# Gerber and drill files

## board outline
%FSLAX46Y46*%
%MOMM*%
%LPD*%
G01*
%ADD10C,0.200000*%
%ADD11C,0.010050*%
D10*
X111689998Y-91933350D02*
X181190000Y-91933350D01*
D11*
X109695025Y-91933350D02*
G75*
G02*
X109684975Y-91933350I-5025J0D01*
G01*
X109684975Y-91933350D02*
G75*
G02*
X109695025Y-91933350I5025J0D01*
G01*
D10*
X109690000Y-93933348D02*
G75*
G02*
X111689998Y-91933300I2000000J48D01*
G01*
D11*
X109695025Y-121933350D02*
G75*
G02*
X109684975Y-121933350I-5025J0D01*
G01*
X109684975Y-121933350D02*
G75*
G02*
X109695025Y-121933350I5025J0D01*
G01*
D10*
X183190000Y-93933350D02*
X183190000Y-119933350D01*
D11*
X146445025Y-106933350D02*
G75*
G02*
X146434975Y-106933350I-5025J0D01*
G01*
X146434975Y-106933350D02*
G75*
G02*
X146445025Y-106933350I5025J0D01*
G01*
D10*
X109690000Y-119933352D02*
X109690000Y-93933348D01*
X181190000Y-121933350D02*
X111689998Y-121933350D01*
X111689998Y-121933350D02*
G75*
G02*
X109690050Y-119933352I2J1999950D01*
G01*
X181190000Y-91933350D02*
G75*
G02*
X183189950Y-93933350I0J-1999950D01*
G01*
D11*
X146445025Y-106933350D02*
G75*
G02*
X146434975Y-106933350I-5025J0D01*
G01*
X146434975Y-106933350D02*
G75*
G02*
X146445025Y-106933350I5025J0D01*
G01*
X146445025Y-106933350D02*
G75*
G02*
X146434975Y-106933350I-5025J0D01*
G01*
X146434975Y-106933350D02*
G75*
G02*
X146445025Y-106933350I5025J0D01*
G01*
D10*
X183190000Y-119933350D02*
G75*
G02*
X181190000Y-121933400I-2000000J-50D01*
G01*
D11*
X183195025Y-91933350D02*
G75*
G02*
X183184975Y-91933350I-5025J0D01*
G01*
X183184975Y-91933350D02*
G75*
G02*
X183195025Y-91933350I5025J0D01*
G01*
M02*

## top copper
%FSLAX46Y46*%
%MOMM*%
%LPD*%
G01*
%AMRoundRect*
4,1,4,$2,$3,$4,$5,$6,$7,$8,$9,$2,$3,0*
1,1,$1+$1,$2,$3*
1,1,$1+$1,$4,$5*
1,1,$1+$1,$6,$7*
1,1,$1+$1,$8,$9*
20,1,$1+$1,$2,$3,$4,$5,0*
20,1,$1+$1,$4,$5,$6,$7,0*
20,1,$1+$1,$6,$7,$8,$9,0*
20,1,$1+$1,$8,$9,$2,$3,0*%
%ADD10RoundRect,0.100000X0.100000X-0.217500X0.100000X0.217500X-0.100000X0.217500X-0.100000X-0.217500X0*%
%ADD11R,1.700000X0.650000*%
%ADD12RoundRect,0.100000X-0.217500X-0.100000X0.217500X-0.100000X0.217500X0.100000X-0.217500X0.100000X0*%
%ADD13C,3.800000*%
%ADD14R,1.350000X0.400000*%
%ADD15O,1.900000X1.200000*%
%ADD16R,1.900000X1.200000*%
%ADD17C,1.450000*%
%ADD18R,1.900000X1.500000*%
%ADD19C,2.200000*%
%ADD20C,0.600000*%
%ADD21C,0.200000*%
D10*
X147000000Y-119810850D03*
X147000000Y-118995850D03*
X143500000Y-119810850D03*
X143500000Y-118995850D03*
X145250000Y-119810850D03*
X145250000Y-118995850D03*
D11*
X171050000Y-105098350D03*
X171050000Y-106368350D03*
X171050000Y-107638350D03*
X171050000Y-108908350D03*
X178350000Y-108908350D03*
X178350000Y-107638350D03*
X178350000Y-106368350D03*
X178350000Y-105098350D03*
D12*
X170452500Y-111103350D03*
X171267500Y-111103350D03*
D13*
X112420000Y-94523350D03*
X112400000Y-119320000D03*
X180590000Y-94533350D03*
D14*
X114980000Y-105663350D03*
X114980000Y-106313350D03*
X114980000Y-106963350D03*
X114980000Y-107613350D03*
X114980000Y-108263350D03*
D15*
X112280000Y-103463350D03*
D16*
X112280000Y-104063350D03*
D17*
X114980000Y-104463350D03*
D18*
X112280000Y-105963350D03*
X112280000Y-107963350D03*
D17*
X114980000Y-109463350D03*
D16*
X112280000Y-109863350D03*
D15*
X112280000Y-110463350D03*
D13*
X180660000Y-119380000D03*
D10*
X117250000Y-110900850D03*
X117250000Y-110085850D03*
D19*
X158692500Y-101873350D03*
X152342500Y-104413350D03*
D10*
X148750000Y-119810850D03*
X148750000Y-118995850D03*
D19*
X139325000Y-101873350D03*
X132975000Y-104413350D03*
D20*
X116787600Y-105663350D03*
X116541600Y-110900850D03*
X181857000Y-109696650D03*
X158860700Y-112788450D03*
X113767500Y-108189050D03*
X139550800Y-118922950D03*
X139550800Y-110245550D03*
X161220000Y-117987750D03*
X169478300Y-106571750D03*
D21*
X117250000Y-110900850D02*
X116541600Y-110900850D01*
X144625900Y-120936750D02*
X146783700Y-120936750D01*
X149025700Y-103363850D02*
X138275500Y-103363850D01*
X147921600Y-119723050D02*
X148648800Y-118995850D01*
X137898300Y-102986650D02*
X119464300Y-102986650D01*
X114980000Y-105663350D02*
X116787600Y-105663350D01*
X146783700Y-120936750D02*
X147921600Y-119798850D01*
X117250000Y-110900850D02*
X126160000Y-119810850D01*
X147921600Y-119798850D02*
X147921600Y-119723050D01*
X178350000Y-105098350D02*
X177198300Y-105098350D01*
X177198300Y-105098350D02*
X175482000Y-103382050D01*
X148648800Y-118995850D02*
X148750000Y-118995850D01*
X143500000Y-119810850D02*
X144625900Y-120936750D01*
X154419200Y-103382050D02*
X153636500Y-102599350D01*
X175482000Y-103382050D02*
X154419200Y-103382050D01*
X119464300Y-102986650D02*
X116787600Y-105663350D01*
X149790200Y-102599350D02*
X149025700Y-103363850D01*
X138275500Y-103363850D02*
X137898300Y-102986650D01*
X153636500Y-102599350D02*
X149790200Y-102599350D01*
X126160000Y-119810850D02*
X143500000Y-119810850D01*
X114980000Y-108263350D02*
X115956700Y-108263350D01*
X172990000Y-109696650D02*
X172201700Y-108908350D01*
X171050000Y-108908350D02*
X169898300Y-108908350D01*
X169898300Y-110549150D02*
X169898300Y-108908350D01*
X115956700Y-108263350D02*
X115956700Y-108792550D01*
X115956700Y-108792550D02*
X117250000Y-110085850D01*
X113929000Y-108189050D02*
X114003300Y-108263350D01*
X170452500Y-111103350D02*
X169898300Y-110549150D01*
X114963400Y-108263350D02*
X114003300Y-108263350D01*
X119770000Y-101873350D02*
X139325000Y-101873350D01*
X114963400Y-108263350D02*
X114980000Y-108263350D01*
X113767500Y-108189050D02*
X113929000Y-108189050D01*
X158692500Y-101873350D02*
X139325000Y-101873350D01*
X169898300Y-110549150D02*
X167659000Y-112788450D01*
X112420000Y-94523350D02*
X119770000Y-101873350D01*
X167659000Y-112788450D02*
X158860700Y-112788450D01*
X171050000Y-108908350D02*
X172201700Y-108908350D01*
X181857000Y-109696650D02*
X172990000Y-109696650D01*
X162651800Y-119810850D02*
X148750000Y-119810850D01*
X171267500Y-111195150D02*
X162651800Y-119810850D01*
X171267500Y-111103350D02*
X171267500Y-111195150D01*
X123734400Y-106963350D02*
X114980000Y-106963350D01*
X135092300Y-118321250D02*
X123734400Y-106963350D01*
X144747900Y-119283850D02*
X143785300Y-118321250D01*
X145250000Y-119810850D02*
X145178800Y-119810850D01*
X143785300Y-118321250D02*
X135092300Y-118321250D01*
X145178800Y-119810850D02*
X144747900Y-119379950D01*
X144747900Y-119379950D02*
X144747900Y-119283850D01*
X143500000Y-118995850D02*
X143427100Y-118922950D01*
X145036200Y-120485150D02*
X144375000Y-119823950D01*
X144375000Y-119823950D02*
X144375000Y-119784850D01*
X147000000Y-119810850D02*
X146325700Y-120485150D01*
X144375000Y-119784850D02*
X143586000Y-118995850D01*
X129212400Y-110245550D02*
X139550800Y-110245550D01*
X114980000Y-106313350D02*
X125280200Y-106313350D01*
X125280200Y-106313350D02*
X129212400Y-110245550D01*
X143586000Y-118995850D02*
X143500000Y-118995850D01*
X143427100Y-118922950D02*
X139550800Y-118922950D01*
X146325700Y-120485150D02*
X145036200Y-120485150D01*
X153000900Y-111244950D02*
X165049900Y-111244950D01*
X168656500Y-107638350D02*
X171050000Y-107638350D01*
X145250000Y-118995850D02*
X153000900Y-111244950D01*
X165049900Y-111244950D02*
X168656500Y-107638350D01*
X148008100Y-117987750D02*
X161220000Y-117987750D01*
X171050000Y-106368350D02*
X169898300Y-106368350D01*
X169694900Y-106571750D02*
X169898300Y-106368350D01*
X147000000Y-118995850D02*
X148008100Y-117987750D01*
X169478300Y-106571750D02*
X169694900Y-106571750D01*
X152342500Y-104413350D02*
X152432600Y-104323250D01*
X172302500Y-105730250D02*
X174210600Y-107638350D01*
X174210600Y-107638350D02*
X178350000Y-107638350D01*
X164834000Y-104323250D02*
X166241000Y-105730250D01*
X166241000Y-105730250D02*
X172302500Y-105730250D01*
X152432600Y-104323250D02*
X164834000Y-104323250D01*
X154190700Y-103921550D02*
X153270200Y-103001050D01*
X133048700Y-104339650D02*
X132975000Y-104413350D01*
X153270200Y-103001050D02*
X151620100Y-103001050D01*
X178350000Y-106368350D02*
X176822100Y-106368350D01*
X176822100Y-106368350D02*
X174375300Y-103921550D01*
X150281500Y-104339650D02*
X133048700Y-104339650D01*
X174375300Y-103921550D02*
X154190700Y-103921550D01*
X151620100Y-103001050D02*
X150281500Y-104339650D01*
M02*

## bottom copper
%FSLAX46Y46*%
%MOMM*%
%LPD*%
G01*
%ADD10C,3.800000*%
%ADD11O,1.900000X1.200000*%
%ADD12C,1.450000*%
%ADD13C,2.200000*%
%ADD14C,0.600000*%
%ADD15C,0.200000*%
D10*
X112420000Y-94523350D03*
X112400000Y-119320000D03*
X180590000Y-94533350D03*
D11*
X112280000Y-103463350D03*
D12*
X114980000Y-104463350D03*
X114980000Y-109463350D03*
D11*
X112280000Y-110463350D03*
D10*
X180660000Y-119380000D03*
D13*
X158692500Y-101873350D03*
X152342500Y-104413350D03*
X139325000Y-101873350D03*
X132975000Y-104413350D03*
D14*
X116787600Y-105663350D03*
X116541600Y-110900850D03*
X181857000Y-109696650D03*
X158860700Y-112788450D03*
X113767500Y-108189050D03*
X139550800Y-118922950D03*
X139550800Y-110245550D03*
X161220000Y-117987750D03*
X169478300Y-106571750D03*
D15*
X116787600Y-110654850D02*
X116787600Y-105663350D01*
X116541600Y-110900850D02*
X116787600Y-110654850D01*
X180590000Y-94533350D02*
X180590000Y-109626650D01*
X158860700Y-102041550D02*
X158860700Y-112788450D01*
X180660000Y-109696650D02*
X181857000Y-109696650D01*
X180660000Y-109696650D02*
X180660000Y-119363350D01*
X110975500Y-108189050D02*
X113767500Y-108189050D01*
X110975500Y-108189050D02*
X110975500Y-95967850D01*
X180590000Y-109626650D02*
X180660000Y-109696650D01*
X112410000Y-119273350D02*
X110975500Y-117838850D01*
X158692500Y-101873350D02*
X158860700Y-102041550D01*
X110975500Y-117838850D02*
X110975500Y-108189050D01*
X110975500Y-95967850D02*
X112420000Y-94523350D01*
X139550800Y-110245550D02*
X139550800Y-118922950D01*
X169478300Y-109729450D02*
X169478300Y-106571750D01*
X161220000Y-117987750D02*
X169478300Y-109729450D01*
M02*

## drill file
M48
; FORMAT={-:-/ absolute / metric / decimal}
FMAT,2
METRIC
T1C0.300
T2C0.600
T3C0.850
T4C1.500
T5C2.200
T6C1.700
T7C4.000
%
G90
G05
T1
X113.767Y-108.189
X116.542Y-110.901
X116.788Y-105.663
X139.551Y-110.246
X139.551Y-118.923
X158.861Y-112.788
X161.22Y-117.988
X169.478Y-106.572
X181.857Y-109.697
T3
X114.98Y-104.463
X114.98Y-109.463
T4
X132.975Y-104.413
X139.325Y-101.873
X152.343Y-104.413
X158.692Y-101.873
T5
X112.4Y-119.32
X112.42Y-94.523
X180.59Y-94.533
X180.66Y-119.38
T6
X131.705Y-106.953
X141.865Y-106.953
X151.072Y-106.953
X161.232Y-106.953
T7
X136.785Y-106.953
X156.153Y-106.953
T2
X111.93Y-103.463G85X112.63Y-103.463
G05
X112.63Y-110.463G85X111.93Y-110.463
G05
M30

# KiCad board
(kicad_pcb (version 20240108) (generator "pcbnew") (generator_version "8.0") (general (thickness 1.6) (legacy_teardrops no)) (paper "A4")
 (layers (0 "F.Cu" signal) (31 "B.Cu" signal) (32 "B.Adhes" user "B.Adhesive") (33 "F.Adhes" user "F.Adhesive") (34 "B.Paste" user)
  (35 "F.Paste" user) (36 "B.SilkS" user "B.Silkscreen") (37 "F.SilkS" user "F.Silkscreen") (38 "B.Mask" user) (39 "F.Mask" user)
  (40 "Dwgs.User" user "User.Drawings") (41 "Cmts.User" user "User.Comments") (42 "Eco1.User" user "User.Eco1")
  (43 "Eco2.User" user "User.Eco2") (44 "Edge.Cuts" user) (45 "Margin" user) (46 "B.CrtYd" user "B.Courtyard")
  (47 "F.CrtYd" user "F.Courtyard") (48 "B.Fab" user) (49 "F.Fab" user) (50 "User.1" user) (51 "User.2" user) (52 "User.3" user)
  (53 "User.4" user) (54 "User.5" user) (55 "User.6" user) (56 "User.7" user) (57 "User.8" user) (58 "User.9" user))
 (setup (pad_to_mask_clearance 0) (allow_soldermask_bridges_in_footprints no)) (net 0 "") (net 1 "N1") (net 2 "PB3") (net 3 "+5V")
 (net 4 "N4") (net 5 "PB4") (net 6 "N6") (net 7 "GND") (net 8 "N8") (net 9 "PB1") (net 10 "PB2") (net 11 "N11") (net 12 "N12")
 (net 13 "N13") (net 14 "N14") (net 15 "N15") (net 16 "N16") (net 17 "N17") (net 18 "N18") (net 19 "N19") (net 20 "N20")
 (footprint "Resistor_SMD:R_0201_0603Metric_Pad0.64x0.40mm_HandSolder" (layer "F.Cu") (at 147 119.40335 90)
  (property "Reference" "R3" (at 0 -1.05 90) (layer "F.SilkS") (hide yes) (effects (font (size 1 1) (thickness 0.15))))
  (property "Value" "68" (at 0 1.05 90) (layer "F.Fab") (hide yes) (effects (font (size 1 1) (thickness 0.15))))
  (pad "" smd roundrect (at -0.4325 0 90) (size 0.458 0.36) (layers "F.Paste") (roundrect_rratio 0.25))
  (pad "" smd roundrect (at 0.4325 0 90) (size 0.458 0.36) (layers "F.Paste") (roundrect_rratio 0.25))
  (pad "1" smd roundrect (at -0.4075 0 90) (size 0.635 0.4) (layers "F.Cu" "F.Mask") (roundrect_rratio 0.25) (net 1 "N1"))
  (pad "2" smd roundrect (at 0.4075 0 90) (size 0.635 0.4) (layers "F.Cu" "F.Mask") (roundrect_rratio 0.25) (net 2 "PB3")))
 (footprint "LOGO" (layer "F.Cu") (at 121.61 121.01)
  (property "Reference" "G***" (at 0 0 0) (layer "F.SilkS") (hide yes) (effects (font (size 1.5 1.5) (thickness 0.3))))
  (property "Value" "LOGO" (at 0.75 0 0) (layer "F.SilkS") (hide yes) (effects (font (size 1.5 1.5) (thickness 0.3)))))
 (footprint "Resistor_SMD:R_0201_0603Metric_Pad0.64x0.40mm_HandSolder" (layer "F.Cu") (at 143.5 119.40335 90)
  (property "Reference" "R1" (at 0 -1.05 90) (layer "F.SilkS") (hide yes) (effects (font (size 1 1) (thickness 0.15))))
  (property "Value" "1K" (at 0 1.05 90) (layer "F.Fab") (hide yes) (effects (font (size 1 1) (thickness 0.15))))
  (pad "" smd roundrect (at -0.4325 0 90) (size 0.458 0.36) (layers "F.Paste") (roundrect_rratio 0.25))
  (pad "" smd roundrect (at 0.4325 0 90) (size 0.458 0.36) (layers "F.Paste") (roundrect_rratio 0.25))
  (pad "1" smd roundrect (at -0.4075 0 90) (size 0.635 0.4) (layers "F.Cu" "F.Mask") (roundrect_rratio 0.25) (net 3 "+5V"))
  (pad "2" smd roundrect (at 0.4075 0 90) (size 0.635 0.4) (layers "F.Cu" "F.Mask") (roundrect_rratio 0.25) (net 1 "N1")))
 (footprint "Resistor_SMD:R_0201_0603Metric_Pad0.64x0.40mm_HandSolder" (layer "F.Cu") (at 145.25 119.40335 90)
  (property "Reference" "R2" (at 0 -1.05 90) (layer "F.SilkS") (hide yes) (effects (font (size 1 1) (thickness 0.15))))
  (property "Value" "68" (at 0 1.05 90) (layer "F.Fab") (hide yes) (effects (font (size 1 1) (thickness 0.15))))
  (pad "" smd roundrect (at -0.4325 0 90) (size 0.458 0.36) (layers "F.Paste") (roundrect_rratio 0.25))
  (pad "" smd roundrect (at 0.4325 0 90) (size 0.458 0.36) (layers "F.Paste") (roundrect_rratio 0.25))
  (pad "1" smd roundrect (at -0.4075 0 90) (size 0.635 0.4) (layers "F.Cu" "F.Mask") (roundrect_rratio 0.25) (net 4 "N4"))
  (pad "2" smd roundrect (at 0.4075 0 90) (size 0.635 0.4) (layers "F.Cu" "F.Mask") (roundrect_rratio 0.25) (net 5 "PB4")))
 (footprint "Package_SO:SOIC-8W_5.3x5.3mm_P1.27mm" (layer "F.Cu") (at 174.7 107.00335)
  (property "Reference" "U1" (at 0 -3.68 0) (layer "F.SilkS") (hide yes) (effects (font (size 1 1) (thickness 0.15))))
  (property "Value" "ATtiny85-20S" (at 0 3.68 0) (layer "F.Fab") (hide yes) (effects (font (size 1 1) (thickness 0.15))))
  (pad "1" smd rect (at -3.65 -1.905) (size 1.7 0.65) (layers "F.Cu" "F.Paste" "F.Mask") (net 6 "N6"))
  (pad "2" smd rect (at -3.65 -0.635) (size 1.7 0.65) (layers "F.Cu" "F.Paste" "F.Mask") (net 2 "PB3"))
  (pad "3" smd rect (at -3.65 0.635) (size 1.7 0.65) (layers "F.Cu" "F.Paste" "F.Mask") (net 5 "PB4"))
  (pad "4" smd rect (at -3.65 1.905) (size 1.7 0.65) (layers "F.Cu" "F.Paste" "F.Mask") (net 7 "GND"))
  (pad "5" smd rect (at 3.65 1.905) (size 1.7 0.65) (layers "F.Cu" "F.Paste" "F.Mask") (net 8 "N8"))
  (pad "6" smd rect (at 3.65 0.635) (size 1.7 0.65) (layers "F.Cu" "F.Paste" "F.Mask") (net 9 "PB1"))
  (pad "7" smd rect (at 3.65 -0.635) (size 1.7 0.65) (layers "F.Cu" "F.Paste" "F.Mask") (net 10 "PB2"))
  (pad "8" smd rect (at 3.65 -1.905) (size 1.7 0.65) (layers "F.Cu" "F.Paste" "F.Mask") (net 3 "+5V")))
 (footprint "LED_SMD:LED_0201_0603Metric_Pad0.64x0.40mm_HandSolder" (layer "F.Cu") (at 170.86 111.10335)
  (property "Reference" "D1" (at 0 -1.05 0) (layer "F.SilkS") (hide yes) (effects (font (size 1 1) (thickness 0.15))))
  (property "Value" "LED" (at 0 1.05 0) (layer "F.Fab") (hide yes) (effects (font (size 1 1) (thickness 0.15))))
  (pad "" smd roundrect (at -0.4325 0) (size 0.458 0.36) (layers "F.Paste") (roundrect_rratio 0.25))
  (pad "" smd roundrect (at 0.4325 0) (size 0.458 0.36) (layers "F.Paste") (roundrect_rratio 0.25))
  (pad "1" smd roundrect (at -0.4075 0) (size 0.635 0.4) (layers "F.Cu" "F.Mask") (roundrect_rratio 0.25) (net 7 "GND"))
  (pad "2" smd roundrect (at 0.4075 0) (size 0.635 0.4) (layers "F.Cu" "F.Mask") (roundrect_rratio 0.25) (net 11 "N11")))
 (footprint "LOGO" (layer "F.Cu") (at 172.42 97.63)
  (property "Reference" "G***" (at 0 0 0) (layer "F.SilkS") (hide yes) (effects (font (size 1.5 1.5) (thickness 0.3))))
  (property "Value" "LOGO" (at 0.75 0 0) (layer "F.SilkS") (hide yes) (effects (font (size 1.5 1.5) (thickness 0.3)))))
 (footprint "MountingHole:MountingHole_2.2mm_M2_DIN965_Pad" (layer "F.Cu") (at 112.42 94.52335)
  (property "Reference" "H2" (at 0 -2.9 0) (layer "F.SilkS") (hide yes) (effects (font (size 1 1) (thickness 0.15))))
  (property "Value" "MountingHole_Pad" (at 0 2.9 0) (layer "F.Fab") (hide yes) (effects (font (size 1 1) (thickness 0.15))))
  (pad "1" thru_hole circle (at 0 0) (size 3.8 3.8) (drill 2.2) (layers "*.Cu" "*.Mask") (remove_unused_layers no) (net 7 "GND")))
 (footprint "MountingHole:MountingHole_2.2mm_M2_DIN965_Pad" (layer "F.Cu") (at 112.4 119.32)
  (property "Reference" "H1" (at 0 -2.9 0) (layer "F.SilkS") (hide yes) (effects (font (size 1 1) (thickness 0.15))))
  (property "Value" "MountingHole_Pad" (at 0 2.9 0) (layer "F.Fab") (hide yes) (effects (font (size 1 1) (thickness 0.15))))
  (pad "1" thru_hole circle (at 0 0) (size 3.8 3.8) (drill 2.2) (layers "*.Cu" "*.Mask") (remove_unused_layers no) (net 7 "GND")))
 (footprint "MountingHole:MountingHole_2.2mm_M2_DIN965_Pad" (layer "F.Cu") (at 180.59 94.53335)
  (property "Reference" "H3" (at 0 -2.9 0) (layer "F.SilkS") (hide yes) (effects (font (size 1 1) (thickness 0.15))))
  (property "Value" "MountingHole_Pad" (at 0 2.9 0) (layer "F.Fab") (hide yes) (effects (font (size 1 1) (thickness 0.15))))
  (pad "1" thru_hole circle (at 0 0) (size 3.8 3.8) (drill 2.2) (layers "*.Cu" "*.Mask") (remove_unused_layers no) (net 7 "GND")))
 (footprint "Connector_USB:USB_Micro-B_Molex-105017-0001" (layer "F.Cu") (at 113.5175 106.96335 -90)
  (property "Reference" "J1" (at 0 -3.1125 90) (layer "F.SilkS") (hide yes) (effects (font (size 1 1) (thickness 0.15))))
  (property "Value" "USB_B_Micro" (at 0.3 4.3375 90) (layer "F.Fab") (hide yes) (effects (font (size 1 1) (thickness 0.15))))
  (pad "1" smd rect (at -1.3 -1.4625 270) (size 0.4 1.35) (layers "F.Cu" "F.Paste" "F.Mask") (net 3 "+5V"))
  (pad "2" smd rect (at -0.65 -1.4625 270) (size 0.4 1.35) (layers "F.Cu" "F.Paste" "F.Mask") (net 1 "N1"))
  (pad "3" smd rect (at 0 -1.4625 270) (size 0.4 1.35) (layers "F.Cu" "F.Paste" "F.Mask") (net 4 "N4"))
  (pad "4" smd rect (at 0.65 -1.4625 270) (size 0.4 1.35) (layers "F.Cu" "F.Paste" "F.Mask") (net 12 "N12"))
  (pad "5" smd rect (at 1.3 -1.4625 270) (size 0.4 1.35) (layers "F.Cu" "F.Paste" "F.Mask") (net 7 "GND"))
  (pad "6" thru_hole oval (at -3.5 1.2375 90) (size 1.2 1.9) (drill oval 0.6 1.3) (layers "*.Cu" "*.Mask") (remove_unused_layers no)
   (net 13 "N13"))
  (pad "6" smd rect (at -2.9 1.2375 270) (size 1.2 1.9) (layers "F.Cu" "F.Mask") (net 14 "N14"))
  (pad "6" thru_hole circle (at -2.5 -1.4625 270) (size 1.45 1.45) (drill 0.85) (layers "*.Cu" "*.Mask") (remove_unused_layers no)
   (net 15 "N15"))
  (pad "6" smd rect (at -1 1.2375 270) (size 1.5 1.9) (layers "F.Cu" "F.Paste" "F.Mask") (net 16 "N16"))
  (pad "6" smd rect (at 1 1.2375 270) (size 1.5 1.9) (layers "F.Cu" "F.Paste" "F.Mask") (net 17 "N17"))
  (pad "6" thru_hole circle (at 2.5 -1.4625 270) (size 1.45 1.45) (drill 0.85) (layers "*.Cu" "*.Mask") (remove_unused_layers no)
   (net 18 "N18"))
  (pad "6" smd rect (at 2.9 1.2375 270) (size 1.2 1.9) (layers "F.Cu" "F.Mask") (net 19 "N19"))
  (pad "6" thru_hole oval (at 3.5 1.2375 270) (size 1.2 1.9) (drill oval 0.6 1.3) (layers "*.Cu" "*.Mask") (remove_unused_layers no)
   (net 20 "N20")))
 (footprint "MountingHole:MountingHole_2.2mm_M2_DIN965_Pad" (layer "F.Cu") (at 180.66 119.38)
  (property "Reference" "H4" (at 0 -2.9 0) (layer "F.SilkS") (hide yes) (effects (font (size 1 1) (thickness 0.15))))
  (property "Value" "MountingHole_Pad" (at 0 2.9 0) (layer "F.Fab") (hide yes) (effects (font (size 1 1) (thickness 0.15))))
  (pad "1" thru_hole circle (at 0 0) (size 3.8 3.8) (drill 2.2) (layers "*.Cu" "*.Mask") (remove_unused_layers no) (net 7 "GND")))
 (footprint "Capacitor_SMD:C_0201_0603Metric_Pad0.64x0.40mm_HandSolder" (layer "F.Cu") (at 117.25 110.49335 90)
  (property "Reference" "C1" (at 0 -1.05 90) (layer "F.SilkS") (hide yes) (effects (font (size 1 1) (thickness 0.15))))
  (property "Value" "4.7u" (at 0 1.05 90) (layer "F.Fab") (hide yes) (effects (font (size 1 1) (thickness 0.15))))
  (pad "" smd roundrect (at -0.4325 0 90) (size 0.458 0.36) (layers "F.Paste") (roundrect_rratio 0.25))
  (pad "" smd roundrect (at 0.4325 0 90) (size 0.458 0.36) (layers "F.Paste") (roundrect_rratio 0.25))
  (pad "1" smd roundrect (at -0.4075 0 90) (size 0.635 0.4) (layers "F.Cu" "F.Mask") (roundrect_rratio 0.25) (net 3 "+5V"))
  (pad "2" smd roundrect (at 0.4075 0 90) (size 0.635 0.4) (layers "F.Cu" "F.Mask") (roundrect_rratio 0.25) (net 7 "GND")))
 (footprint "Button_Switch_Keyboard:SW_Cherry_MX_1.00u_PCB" (layer "F.Cu") (at 158.6925 101.87335)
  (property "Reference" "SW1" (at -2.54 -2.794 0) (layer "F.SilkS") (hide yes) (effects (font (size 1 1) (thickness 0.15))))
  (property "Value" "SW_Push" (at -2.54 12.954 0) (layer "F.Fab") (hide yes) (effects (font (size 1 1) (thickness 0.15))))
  (pad "" np_thru_hole circle (at -7.62 5.08) (size 1.7 1.7) (drill 1.7) (layers "*.Cu" "*.Mask"))
  (pad "" np_thru_hole circle (at -2.54 5.08) (size 4 4) (drill 4) (layers "*.Cu" "*.Mask"))
  (pad "" np_thru_hole circle (at 2.54 5.08) (size 1.7 1.7) (drill 1.7) (layers "*.Cu" "*.Mask"))
  (pad "1" thru_hole circle (at 0 0) (size 2.2 2.2) (drill 1.5) (layers "*.Cu" "*.Mask") (remove_unused_layers no) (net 7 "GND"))
  (pad "2" thru_hole circle (at -6.35 2.54) (size 2.2 2.2) (drill 1.5) (layers "*.Cu" "*.Mask") (remove_unused_layers no) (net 9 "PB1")))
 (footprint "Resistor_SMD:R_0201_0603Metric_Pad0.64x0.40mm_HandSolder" (layer "F.Cu") (at 148.75 119.40335 90)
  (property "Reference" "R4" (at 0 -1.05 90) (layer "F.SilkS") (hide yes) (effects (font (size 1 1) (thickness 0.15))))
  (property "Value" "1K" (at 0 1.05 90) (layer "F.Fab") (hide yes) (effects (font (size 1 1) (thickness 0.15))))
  (pad "" smd roundrect (at -0.4325 0 90) (size 0.458 0.36) (layers "F.Paste") (roundrect_rratio 0.25))
  (pad "" smd roundrect (at 0.4325 0 90) (size 0.458 0.36) (layers "F.Paste") (roundrect_rratio 0.25))
  (pad "1" smd roundrect (at -0.4075 0 90) (size 0.635 0.4) (layers "F.Cu" "F.Mask") (roundrect_rratio 0.25) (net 11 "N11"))
  (pad "2" smd roundrect (at 0.4075 0 90) (size 0.635 0.4) (layers "F.Cu" "F.Mask") (roundrect_rratio 0.25) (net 3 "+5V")))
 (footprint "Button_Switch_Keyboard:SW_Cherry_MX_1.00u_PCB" (layer "F.Cu") (at 139.325 101.87335)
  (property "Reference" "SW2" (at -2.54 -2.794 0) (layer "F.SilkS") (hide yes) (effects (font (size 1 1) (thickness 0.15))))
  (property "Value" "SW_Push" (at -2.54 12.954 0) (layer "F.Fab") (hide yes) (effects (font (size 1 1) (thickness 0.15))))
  (pad "" np_thru_hole circle (at -7.62 5.08) (size 1.7 1.7) (drill 1.7) (layers "*.Cu" "*.Mask"))
  (pad "" np_thru_hole circle (at -2.54 5.08) (size 4 4) (drill 4) (layers "*.Cu" "*.Mask"))
  (pad "" np_thru_hole circle (at 2.54 5.08) (size 1.7 1.7) (drill 1.7) (layers "*.Cu" "*.Mask"))
  (pad "1" thru_hole circle (at 0 0) (size 2.2 2.2) (drill 1.5) (layers "*.Cu" "*.Mask") (remove_unused_layers no) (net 7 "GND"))
  (pad "2" thru_hole circle (at -6.35 2.54) (size 2.2 2.2) (drill 1.5) (layers "*.Cu" "*.Mask") (remove_unused_layers no) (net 10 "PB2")))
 (gr_line (start 111.689998 91.93335) (end 181.19 91.93335) (stroke (width 0.2) (type default)) (layer "Edge.Cuts"))
 (gr_circle (center 109.69 91.93335) (end 109.7 91.93335) (stroke (width 0.0001) (type default)) (fill solid) (layer "Edge.Cuts"))
 (gr_arc (start 109.69 93.933348) (mid 110.275786 92.519136) (end 111.689998 91.93335) (stroke (width 0.2) (type default))
  (layer "Edge.Cuts"))
 (gr_circle (center 109.69 121.93335) (end 109.7 121.93335) (stroke (width 0.0001) (type default)) (fill solid) (layer "Edge.Cuts"))
 (gr_line (start 183.19 93.93335) (end 183.19 119.93335) (stroke (width 0.2) (type default)) (layer "Edge.Cuts"))
 (gr_circle (center 146.44 106.93335) (end 146.45 106.93335) (stroke (width 0.0001) (type default)) (fill solid) (layer "Edge.Cuts"))
 (gr_line (start 109.69 119.933352) (end 109.69 93.933348) (stroke (width 0.2) (type default)) (layer "Edge.Cuts"))
 (gr_line (start 181.19 121.93335) (end 111.689998 121.93335) (stroke (width 0.2) (type default)) (layer "Edge.Cuts"))
 (gr_arc (start 111.689998 121.93335) (mid 110.275786 121.347564) (end 109.69 119.933352) (stroke (width 0.2) (type default))
  (layer "Edge.Cuts"))
 (gr_arc (start 181.19 91.93335) (mid 182.604214 92.519136) (end 183.19 93.93335) (stroke (width 0.2) (type default)) (layer "Edge.Cuts"))
 (gr_circle (center 146.44 106.93335) (end 146.45 106.93335) (stroke (width 0.0001) (type default)) (fill solid) (layer "Edge.Cuts"))
 (gr_circle (center 146.44 106.93335) (end 146.45 106.93335) (stroke (width 0.0001) (type default)) (fill solid) (layer "Edge.Cuts"))
 (gr_arc (start 183.19 119.93335) (mid 182.604214 121.347564) (end 181.19 121.93335) (stroke (width 0.2) (type default)) (layer "Edge.Cuts"))
 (gr_circle (center 183.19 91.93335) (end 183.2 91.93335) (stroke (width 0.0001) (type default)) (fill solid) (layer "Edge.Cuts"))
 (segment (start 117.25 110.90085) (end 116.5416 110.90085) (width 0.2) (layer "F.Cu") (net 3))
 (segment (start 144.6259 120.93675) (end 146.7837 120.93675) (width 0.2) (layer "F.Cu") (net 3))
 (segment (start 149.0257 103.36385) (end 138.2755 103.36385) (width 0.2) (layer "F.Cu") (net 3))
 (segment (start 147.9216 119.72305) (end 148.6488 118.99585) (width 0.2) (layer "F.Cu") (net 3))
 (segment (start 137.8983 102.98665) (end 119.4643 102.98665) (width 0.2) (layer "F.Cu") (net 3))
 (segment (start 114.98 105.66335) (end 116.7876 105.66335) (width 0.2) (layer "F.Cu") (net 3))
 (segment (start 146.7837 120.93675) (end 147.9216 119.79885) (width 0.2) (layer "F.Cu") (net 3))
 (segment (start 117.25 110.90085) (end 126.16 119.81085) (width 0.2) (layer "F.Cu") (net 3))
 (segment (start 147.9216 119.79885) (end 147.9216 119.72305) (width 0.2) (layer "F.Cu") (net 3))
 (segment (start 178.35 105.09835) (end 177.1983 105.09835) (width 0.2) (layer "F.Cu") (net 3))
 (segment (start 177.1983 105.09835) (end 175.482 103.38205) (width 0.2) (layer "F.Cu") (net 3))
 (segment (start 148.6488 118.99585) (end 148.75 118.99585) (width 0.2) (layer "F.Cu") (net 3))
 (segment (start 143.5 119.81085) (end 144.6259 120.93675) (width 0.2) (layer "F.Cu") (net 3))
 (segment (start 154.4192 103.38205) (end 153.6365 102.59935) (width 0.2) (layer "F.Cu") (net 3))
 (segment (start 175.482 103.38205) (end 154.4192 103.38205) (width 0.2) (layer "F.Cu") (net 3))
 (segment (start 119.4643 102.98665) (end 116.7876 105.66335) (width 0.2) (layer "F.Cu") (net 3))
 (segment (start 149.7902 102.59935) (end 149.0257 103.36385) (width 0.2) (layer "F.Cu") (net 3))
 (segment (start 138.2755 103.36385) (end 137.8983 102.98665) (width 0.2) (layer "F.Cu") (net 3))
 (segment (start 153.6365 102.59935) (end 149.7902 102.59935) (width 0.2) (layer "F.Cu") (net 3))
 (segment (start 126.16 119.81085) (end 143.5 119.81085) (width 0.2) (layer "F.Cu") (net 3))
 (via (at 116.7876 105.66335) (size 0.6) (drill 0.3) (layers "F.Cu" "B.Cu") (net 3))
 (via (at 116.5416 110.90085) (size 0.6) (drill 0.3) (layers "F.Cu" "B.Cu") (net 3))
 (segment (start 116.7876 110.65485) (end 116.7876 105.66335) (width 0.2) (layer "B.Cu") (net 3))
 (segment (start 116.5416 110.90085) (end 116.7876 110.65485) (width 0.2) (layer "B.Cu") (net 3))
 (segment (start 114.98 108.26335) (end 115.9567 108.26335) (width 0.2) (layer "F.Cu") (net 7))
 (segment (start 172.99 109.69665) (end 172.2017 108.90835) (width 0.2) (layer "F.Cu") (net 7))
 (segment (start 171.05 108.90835) (end 169.8983 108.90835) (width 0.2) (layer "F.Cu") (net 7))
 (segment (start 169.8983 110.54915) (end 169.8983 108.90835) (width 0.2) (layer "F.Cu") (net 7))
 (segment (start 115.9567 108.26335) (end 115.9567 108.79255) (width 0.2) (layer "F.Cu") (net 7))
 (segment (start 115.9567 108.79255) (end 117.25 110.08585) (width 0.2) (layer "F.Cu") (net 7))
 (segment (start 113.929 108.18905) (end 114.0033 108.26335) (width 0.2) (layer "F.Cu") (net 7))
 (segment (start 170.4525 111.10335) (end 169.8983 110.54915) (width 0.2) (layer "F.Cu") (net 7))
 (segment (start 114.9634 108.26335) (end 114.0033 108.26335) (width 0.2) (layer "F.Cu") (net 7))
 (segment (start 119.77 101.87335) (end 139.325 101.87335) (width 0.2) (layer "F.Cu") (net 7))
 (segment (start 114.9634 108.26335) (end 114.98 108.26335) (width 0.2) (layer "F.Cu") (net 7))
 (segment (start 113.7675 108.18905) (end 113.929 108.18905) (width 0.2) (layer "F.Cu") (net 7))
 (segment (start 158.6925 101.87335) (end 139.325 101.87335) (width 0.2) (layer "F.Cu") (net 7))
 (segment (start 169.8983 110.54915) (end 167.659 112.78845) (width 0.2) (layer "F.Cu") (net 7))
 (segment (start 112.42 94.52335) (end 119.77 101.87335) (width 0.2) (layer "F.Cu") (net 7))
 (segment (start 167.659 112.78845) (end 158.8607 112.78845) (width 0.2) (layer "F.Cu") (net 7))
 (segment (start 171.05 108.90835) (end 172.2017 108.90835) (width 0.2) (layer "F.Cu") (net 7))
 (segment (start 181.857 109.69665) (end 172.99 109.69665) (width 0.2) (layer "F.Cu") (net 7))
 (via (at 181.857 109.69665) (size 0.6) (drill 0.3) (layers "F.Cu" "B.Cu") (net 7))
 (via (at 158.8607 112.78845) (size 0.6) (drill 0.3) (layers "F.Cu" "B.Cu") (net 7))
 (via (at 113.7675 108.18905) (size 0.6) (drill 0.3) (layers "F.Cu" "B.Cu") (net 7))
 (segment (start 180.59 94.53335) (end 180.59 109.62665) (width 0.2) (layer "B.Cu") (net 7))
 (segment (start 158.8607 102.04155) (end 158.8607 112.78845) (width 0.2) (layer "B.Cu") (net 7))
 (segment (start 180.66 109.69665) (end 181.857 109.69665) (width 0.2) (layer "B.Cu") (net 7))
 (segment (start 180.66 109.69665) (end 180.66 119.36335) (width 0.2) (layer "B.Cu") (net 7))
 (segment (start 110.9755 108.18905) (end 113.7675 108.18905) (width 0.2) (layer "B.Cu") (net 7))
 (segment (start 110.9755 108.18905) (end 110.9755 95.96785) (width 0.2) (layer "B.Cu") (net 7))
 (segment (start 180.59 109.62665) (end 180.66 109.69665) (width 0.2) (layer "B.Cu") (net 7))
 (segment (start 112.41 119.27335) (end 110.9755 117.83885) (width 0.2) (layer "B.Cu") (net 7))
 (segment (start 158.6925 101.87335) (end 158.8607 102.04155) (width 0.2) (layer "B.Cu") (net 7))
 (segment (start 110.9755 117.83885) (end 110.9755 108.18905) (width 0.2) (layer "B.Cu") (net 7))
 (segment (start 110.9755 95.96785) (end 112.42 94.52335) (width 0.2) (layer "B.Cu") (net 7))
 (segment (start 162.6518 119.81085) (end 148.75 119.81085) (width 0.2) (layer "F.Cu") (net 11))
 (segment (start 171.2675 111.19515) (end 162.6518 119.81085) (width 0.2) (layer "F.Cu") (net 11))
 (segment (start 171.2675 111.10335) (end 171.2675 111.19515) (width 0.2) (layer "F.Cu") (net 11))
 (segment (start 123.7344 106.96335) (end 114.98 106.96335) (width 0.2) (layer "F.Cu") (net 4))
 (segment (start 135.0923 118.32125) (end 123.7344 106.96335) (width 0.2) (layer "F.Cu") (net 4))
 (segment (start 144.7479 119.28385) (end 143.7853 118.32125) (width 0.2) (layer "F.Cu") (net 4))
 (segment (start 145.25 119.81085) (end 145.1788 119.81085) (width 0.2) (layer "F.Cu") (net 4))
 (segment (start 143.7853 118.32125) (end 135.0923 118.32125) (width 0.2) (layer "F.Cu") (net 4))
 (segment (start 145.1788 119.81085) (end 144.7479 119.37995) (width 0.2) (layer "F.Cu") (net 4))
 (segment (start 144.7479 119.37995) (end 144.7479 119.28385) (width 0.2) (layer "F.Cu") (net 4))
 (segment (start 143.5 118.99585) (end 143.4271 118.92295) (width 0.2) (layer "F.Cu") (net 1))
 (segment (start 145.0362 120.48515) (end 144.375 119.82395) (width 0.2) (layer "F.Cu") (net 1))
 (segment (start 144.375 119.82395) (end 144.375 119.78485) (width 0.2) (layer "F.Cu") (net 1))
 (segment (start 147 119.81085) (end 146.3257 120.48515) (width 0.2) (layer "F.Cu") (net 1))
 (segment (start 144.375 119.78485) (end 143.586 118.99585) (width 0.2) (layer "F.Cu") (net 1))
 (segment (start 129.2124 110.24555) (end 139.5508 110.24555) (width 0.2) (layer "F.Cu") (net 1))
 (segment (start 114.98 106.31335) (end 125.2802 106.31335) (width 0.2) (layer "F.Cu") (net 1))
 (segment (start 125.2802 106.31335) (end 129.2124 110.24555) (width 0.2) (layer "F.Cu") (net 1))
 (segment (start 143.586 118.99585) (end 143.5 118.99585) (width 0.2) (layer "F.Cu") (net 1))
 (segment (start 143.4271 118.92295) (end 139.5508 118.92295) (width 0.2) (layer "F.Cu") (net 1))
 (segment (start 146.3257 120.48515) (end 145.0362 120.48515) (width 0.2) (layer "F.Cu") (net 1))
 (via (at 139.5508 118.92295) (size 0.6) (drill 0.3) (layers "F.Cu" "B.Cu") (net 1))
 (via (at 139.5508 110.24555) (size 0.6) (drill 0.3) (layers "F.Cu" "B.Cu") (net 1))
 (segment (start 139.5508 110.24555) (end 139.5508 118.92295) (width 0.2) (layer "B.Cu") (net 1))
 (segment (start 153.0009 111.24495) (end 165.0499 111.24495) (width 0.2) (layer "F.Cu") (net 5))
 (segment (start 168.6565 107.63835) (end 171.05 107.63835) (width 0.2) (layer "F.Cu") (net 5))
 (segment (start 145.25 118.99585) (end 153.0009 111.24495) (width 0.2) (layer "F.Cu") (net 5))
 (segment (start 165.0499 111.24495) (end 168.6565 107.63835) (width 0.2) (layer "F.Cu") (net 5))
 (segment (start 148.0081 117.98775) (end 161.22 117.98775) (width 0.2) (layer "F.Cu") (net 2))
 (segment (start 171.05 106.36835) (end 169.8983 106.36835) (width 0.2) (layer "F.Cu") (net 2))
 (segment (start 169.6949 106.57175) (end 169.8983 106.36835) (width 0.2) (layer "F.Cu") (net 2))
 (segment (start 147 118.99585) (end 148.0081 117.98775) (width 0.2) (layer "F.Cu") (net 2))
 (segment (start 169.4783 106.57175) (end 169.6949 106.57175) (width 0.2) (layer "F.Cu") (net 2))
 (via (at 161.22 117.98775) (size 0.6) (drill 0.3) (layers "F.Cu" "B.Cu") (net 2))
 (via (at 169.4783 106.57175) (size 0.6) (drill 0.3) (layers "F.Cu" "B.Cu") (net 2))
 (segment (start 169.4783 109.72945) (end 169.4783 106.57175) (width 0.2) (layer "B.Cu") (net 2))
 (segment (start 161.22 117.98775) (end 169.4783 109.72945) (width 0.2) (layer "B.Cu") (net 2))
 (segment (start 152.3425 104.41335) (end 152.4326 104.32325) (width 0.2) (layer "F.Cu") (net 9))
 (segment (start 172.3025 105.73025) (end 174.2106 107.63835) (width 0.2) (layer "F.Cu") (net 9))
 (segment (start 174.2106 107.63835) (end 178.35 107.63835) (width 0.2) (layer "F.Cu") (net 9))
 (segment (start 164.834 104.32325) (end 166.241 105.73025) (width 0.2) (layer "F.Cu") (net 9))
 (segment (start 166.241 105.73025) (end 172.3025 105.73025) (width 0.2) (layer "F.Cu") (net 9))
 (segment (start 152.4326 104.32325) (end 164.834 104.32325) (width 0.2) (layer "F.Cu") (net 9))
 (segment (start 154.1907 103.92155) (end 153.2702 103.00105) (width 0.2) (layer "F.Cu") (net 10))
 (segment (start 133.0487 104.33965) (end 132.975 104.41335) (width 0.2) (layer "F.Cu") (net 10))
 (segment (start 153.2702 103.00105) (end 151.6201 103.00105) (width 0.2) (layer "F.Cu") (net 10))
 (segment (start 178.35 106.36835) (end 176.8221 106.36835) (width 0.2) (layer "F.Cu") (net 10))
 (segment (start 176.8221 106.36835) (end 174.3753 103.92155) (width 0.2) (layer "F.Cu") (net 10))
 (segment (start 150.2815 104.33965) (end 133.0487 104.33965) (width 0.2) (layer "F.Cu") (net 10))
 (segment (start 174.3753 103.92155) (end 154.1907 103.92155) (width 0.2) (layer "F.Cu") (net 10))
 (segment (start 151.6201 103.00105) (end 150.2815 104.33965) (width 0.2) (layer "F.Cu") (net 10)))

